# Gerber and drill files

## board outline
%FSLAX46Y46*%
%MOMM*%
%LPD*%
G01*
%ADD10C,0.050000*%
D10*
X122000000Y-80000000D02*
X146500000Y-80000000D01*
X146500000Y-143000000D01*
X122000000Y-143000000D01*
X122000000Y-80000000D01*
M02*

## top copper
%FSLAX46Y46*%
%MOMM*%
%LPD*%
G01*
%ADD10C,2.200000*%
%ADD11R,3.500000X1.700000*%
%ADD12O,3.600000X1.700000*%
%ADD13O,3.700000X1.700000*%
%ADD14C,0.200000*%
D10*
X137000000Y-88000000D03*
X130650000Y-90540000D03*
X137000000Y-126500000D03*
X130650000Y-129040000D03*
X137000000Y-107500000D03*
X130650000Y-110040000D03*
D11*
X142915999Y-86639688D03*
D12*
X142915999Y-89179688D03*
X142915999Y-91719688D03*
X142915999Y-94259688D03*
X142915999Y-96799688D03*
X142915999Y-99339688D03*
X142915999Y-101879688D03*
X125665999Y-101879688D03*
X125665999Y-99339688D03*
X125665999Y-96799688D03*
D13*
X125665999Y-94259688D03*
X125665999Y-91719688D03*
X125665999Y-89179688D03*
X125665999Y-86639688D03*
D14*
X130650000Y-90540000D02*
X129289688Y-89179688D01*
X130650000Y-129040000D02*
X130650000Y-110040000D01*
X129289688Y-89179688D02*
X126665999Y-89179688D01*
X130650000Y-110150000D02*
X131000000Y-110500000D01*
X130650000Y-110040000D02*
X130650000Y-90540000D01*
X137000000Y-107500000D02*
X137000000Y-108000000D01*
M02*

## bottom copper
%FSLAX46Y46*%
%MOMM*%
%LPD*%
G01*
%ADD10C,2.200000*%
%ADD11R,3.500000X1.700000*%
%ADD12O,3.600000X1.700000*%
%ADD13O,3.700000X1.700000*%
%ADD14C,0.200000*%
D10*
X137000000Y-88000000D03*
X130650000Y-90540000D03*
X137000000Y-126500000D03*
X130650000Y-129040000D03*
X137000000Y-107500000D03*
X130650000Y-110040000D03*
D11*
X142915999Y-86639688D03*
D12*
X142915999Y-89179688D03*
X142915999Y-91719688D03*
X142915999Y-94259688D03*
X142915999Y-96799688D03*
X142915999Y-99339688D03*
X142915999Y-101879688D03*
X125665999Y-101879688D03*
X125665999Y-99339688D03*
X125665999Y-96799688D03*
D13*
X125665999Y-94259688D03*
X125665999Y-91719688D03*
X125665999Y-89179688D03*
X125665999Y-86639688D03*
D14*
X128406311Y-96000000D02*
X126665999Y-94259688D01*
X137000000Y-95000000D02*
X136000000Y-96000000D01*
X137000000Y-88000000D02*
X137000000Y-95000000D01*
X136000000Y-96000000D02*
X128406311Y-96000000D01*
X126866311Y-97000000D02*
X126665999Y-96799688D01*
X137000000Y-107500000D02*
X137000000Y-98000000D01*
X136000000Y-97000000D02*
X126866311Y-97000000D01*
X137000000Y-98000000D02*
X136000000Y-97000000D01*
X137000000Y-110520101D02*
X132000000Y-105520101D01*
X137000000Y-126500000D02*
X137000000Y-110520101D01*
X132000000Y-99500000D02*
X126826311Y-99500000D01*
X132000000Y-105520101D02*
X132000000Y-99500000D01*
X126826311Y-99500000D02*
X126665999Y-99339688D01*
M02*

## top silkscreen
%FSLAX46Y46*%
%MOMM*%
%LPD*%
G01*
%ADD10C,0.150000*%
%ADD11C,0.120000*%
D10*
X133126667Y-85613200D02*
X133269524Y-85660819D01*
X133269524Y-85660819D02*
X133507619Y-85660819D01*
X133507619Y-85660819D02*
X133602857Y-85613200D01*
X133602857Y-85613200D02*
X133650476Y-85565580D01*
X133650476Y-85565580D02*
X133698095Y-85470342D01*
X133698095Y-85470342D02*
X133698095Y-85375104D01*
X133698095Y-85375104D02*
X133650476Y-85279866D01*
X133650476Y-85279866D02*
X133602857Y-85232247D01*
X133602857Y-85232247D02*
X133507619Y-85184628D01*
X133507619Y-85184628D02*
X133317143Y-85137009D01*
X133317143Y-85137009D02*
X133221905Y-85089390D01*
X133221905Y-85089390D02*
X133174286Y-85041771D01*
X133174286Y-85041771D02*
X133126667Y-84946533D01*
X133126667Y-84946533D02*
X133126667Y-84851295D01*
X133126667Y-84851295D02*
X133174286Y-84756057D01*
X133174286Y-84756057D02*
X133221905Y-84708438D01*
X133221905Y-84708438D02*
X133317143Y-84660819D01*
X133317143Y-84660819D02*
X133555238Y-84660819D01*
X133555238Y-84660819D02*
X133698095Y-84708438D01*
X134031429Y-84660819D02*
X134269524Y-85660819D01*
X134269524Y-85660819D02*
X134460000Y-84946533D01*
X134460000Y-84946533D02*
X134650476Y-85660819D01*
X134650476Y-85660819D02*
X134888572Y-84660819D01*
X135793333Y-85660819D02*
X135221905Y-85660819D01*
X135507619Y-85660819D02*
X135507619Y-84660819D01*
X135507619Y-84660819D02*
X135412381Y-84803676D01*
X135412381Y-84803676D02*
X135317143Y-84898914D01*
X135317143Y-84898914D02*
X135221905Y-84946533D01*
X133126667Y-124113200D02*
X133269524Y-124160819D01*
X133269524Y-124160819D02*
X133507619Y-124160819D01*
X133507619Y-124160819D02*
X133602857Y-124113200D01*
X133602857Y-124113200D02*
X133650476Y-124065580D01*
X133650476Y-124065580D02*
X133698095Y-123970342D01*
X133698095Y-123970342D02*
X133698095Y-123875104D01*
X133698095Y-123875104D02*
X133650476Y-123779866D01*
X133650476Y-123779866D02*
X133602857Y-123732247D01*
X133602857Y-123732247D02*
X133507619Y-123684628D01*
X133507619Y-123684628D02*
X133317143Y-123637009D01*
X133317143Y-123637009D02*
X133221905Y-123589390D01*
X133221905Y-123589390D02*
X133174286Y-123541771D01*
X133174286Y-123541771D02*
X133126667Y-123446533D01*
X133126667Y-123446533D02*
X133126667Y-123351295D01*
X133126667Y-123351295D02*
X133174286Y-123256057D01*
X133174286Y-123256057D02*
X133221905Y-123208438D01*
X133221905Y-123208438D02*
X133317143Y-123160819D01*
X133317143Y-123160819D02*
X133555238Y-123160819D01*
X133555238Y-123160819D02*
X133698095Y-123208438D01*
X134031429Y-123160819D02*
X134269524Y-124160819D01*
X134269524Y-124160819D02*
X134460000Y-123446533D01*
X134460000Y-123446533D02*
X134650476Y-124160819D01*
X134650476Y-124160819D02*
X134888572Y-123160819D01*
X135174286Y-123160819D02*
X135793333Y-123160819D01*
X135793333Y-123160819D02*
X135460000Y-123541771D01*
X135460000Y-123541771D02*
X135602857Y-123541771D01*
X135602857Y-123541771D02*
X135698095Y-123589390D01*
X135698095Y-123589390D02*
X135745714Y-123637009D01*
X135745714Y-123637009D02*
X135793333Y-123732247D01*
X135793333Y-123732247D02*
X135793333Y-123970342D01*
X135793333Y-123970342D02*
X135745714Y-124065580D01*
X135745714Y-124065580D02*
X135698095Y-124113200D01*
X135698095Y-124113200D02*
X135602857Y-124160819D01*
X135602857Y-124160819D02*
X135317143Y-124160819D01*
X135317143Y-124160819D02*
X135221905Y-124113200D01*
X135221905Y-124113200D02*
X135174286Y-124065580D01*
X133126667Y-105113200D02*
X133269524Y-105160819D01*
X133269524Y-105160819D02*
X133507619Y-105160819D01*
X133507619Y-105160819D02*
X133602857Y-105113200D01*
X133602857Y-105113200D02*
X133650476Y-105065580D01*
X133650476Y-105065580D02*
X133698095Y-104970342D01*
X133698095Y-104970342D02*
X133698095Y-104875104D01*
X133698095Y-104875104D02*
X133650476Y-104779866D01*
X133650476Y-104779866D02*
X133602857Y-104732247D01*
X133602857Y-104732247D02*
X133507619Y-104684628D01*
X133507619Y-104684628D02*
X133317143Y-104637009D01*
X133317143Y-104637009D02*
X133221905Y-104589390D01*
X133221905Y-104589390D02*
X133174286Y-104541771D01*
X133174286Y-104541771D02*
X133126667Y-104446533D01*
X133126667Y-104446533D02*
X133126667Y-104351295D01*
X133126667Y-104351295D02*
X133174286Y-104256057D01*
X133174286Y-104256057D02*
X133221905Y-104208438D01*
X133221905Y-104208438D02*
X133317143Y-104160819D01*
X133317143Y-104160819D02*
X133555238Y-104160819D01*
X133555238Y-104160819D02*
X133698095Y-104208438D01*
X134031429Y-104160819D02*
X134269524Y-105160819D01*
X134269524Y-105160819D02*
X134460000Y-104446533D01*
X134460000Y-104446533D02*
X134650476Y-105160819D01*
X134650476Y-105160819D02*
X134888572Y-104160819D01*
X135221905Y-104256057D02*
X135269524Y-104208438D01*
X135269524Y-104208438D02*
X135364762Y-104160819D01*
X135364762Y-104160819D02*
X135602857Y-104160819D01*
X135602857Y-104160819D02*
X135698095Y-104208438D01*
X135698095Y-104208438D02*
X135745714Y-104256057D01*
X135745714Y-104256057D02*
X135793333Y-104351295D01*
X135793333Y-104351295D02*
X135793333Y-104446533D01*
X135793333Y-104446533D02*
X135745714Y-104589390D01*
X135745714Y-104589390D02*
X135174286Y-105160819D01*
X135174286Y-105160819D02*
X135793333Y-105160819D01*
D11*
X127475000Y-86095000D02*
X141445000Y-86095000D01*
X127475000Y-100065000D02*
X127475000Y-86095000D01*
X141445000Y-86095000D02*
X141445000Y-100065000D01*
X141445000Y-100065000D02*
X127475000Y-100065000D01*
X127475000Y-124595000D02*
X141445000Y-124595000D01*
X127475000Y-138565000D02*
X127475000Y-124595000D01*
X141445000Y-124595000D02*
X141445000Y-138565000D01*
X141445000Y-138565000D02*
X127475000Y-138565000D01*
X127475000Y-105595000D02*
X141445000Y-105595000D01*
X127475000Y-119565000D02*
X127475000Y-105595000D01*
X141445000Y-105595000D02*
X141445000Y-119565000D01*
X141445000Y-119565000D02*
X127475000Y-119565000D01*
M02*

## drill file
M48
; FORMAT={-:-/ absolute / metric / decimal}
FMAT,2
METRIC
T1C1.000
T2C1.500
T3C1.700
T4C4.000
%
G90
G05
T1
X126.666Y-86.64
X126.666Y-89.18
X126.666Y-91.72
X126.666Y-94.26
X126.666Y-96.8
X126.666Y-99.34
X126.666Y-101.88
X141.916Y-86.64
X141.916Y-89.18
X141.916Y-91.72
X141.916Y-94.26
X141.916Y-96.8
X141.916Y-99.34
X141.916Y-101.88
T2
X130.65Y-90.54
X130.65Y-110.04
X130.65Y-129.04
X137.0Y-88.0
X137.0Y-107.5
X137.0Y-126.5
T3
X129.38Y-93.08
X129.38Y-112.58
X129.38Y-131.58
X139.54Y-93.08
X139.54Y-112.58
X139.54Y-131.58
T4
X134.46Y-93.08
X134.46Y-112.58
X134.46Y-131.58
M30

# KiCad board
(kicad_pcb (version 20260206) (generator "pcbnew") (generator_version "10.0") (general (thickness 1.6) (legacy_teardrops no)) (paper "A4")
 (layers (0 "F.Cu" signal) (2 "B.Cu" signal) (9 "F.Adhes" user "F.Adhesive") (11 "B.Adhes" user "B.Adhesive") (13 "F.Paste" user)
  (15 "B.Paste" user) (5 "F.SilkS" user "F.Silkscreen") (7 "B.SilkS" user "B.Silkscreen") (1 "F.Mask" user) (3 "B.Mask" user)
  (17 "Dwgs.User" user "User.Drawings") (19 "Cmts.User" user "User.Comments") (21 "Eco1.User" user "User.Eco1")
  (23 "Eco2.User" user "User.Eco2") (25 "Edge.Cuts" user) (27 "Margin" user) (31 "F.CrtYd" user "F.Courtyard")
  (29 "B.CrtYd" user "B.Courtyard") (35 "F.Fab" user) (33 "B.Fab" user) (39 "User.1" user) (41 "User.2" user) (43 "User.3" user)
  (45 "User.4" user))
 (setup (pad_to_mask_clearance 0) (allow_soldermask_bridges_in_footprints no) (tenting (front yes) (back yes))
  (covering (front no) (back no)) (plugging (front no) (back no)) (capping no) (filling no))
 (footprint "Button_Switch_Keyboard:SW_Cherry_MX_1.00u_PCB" (layer "F.Cu") (at 137 88)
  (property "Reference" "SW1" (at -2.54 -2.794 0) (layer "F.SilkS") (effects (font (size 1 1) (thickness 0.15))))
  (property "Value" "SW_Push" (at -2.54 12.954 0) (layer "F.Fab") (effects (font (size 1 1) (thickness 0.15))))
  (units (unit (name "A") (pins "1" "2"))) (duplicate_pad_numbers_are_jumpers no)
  (fp_line (start -9.525 -1.905) (end 4.445 -1.905) (stroke (width 0.12) (type solid)) (layer "F.SilkS"))
  (fp_line (start -9.525 12.065) (end -9.525 -1.905) (stroke (width 0.12) (type solid)) (layer "F.SilkS"))
  (fp_line (start 4.445 -1.905) (end 4.445 12.065) (stroke (width 0.12) (type solid)) (layer "F.SilkS"))
  (fp_line (start 4.445 12.065) (end -9.525 12.065) (stroke (width 0.12) (type solid)) (layer "F.SilkS"))
  (pad "" np_thru_hole circle (at -7.62 5.08) (size 1.7 1.7) (drill 1.7) (layers "*.Cu" "*.Mask"))
  (pad "" np_thru_hole circle (at -2.54 5.08) (size 4 4) (drill 4) (layers "*.Cu" "*.Mask"))
  (pad "" np_thru_hole circle (at 2.54 5.08) (size 1.7 1.7) (drill 1.7) (layers "*.Cu" "*.Mask"))
  (pad "1" thru_hole circle (at 0 0) (size 2.2 2.2) (drill 1.5) (layers "*.Cu" "*.Mask") (remove_unused_layers no)
   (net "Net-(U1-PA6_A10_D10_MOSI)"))
  (pad "2" thru_hole circle (at -6.35 2.54) (size 2.2 2.2) (drill 1.5) (layers "*.Cu" "*.Mask") (remove_unused_layers no) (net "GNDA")))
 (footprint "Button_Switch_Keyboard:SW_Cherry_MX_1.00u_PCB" (layer "F.Cu") (at 137 126.5)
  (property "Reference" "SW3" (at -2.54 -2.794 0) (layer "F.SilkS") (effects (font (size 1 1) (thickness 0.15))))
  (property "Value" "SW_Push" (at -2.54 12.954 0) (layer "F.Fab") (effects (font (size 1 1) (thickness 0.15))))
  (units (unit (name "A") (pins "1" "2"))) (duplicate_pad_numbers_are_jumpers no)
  (fp_line (start -9.525 -1.905) (end 4.445 -1.905) (stroke (width 0.12) (type solid)) (layer "F.SilkS"))
  (fp_line (start -9.525 12.065) (end -9.525 -1.905) (stroke (width 0.12) (type solid)) (layer "F.SilkS"))
  (fp_line (start 4.445 -1.905) (end 4.445 12.065) (stroke (width 0.12) (type solid)) (layer "F.SilkS"))
  (fp_line (start 4.445 12.065) (end -9.525 12.065) (stroke (width 0.12) (type solid)) (layer "F.SilkS"))
  (pad "" np_thru_hole circle (at -7.62 5.08) (size 1.7 1.7) (drill 1.7) (layers "*.Cu" "*.Mask"))
  (pad "" np_thru_hole circle (at -2.54 5.08) (size 4 4) (drill 4) (layers "*.Cu" "*.Mask"))
  (pad "" np_thru_hole circle (at 2.54 5.08) (size 1.7 1.7) (drill 1.7) (layers "*.Cu" "*.Mask"))
  (pad "1" thru_hole circle (at 0 0) (size 2.2 2.2) (drill 1.5) (layers "*.Cu" "*.Mask") (remove_unused_layers no)
   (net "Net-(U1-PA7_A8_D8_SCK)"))
  (pad "2" thru_hole circle (at -6.35 2.54) (size 2.2 2.2) (drill 1.5) (layers "*.Cu" "*.Mask") (remove_unused_layers no) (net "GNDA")))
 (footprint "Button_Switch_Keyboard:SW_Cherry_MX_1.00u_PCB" (layer "F.Cu") (at 137 107.5)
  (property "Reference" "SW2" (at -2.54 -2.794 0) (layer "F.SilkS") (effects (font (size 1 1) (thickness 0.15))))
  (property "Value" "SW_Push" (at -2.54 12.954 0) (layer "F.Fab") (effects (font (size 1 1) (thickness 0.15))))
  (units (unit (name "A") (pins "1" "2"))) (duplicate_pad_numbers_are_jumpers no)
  (fp_line (start -9.525 -1.905) (end 4.445 -1.905) (stroke (width 0.12) (type solid)) (layer "F.SilkS"))
  (fp_line (start -9.525 12.065) (end -9.525 -1.905) (stroke (width 0.12) (type solid)) (layer "F.SilkS"))
  (fp_line (start 4.445 -1.905) (end 4.445 12.065) (stroke (width 0.12) (type solid)) (layer "F.SilkS"))
  (fp_line (start 4.445 12.065) (end -9.525 12.065) (stroke (width 0.12) (type solid)) (layer "F.SilkS"))
  (pad "" np_thru_hole circle (at -7.62 5.08) (size 1.7 1.7) (drill 1.7) (layers "*.Cu" "*.Mask"))
  (pad "" np_thru_hole circle (at -2.54 5.08) (size 4 4) (drill 4) (layers "*.Cu" "*.Mask"))
  (pad "" np_thru_hole circle (at 2.54 5.08) (size 1.7 1.7) (drill 1.7) (layers "*.Cu" "*.Mask"))
  (pad "1" thru_hole circle (at 0 0) (size 2.2 2.2) (drill 1.5) (layers "*.Cu" "*.Mask") (remove_unused_layers no)
   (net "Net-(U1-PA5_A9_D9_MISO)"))
  (pad "2" thru_hole circle (at -6.35 2.54) (size 2.2 2.2) (drill 1.5) (layers "*.Cu" "*.Mask") (remove_unused_layers no) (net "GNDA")))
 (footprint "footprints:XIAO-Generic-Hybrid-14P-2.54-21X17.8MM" (layer "B.Cu") (at 134.290999 94.259688 180)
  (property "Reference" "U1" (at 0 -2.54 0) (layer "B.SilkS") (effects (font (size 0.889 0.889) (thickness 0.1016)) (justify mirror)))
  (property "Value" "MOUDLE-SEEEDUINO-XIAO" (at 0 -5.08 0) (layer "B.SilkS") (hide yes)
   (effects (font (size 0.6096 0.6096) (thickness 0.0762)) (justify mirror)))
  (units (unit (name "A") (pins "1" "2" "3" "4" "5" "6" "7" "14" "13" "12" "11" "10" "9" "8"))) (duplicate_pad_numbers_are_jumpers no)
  (pad "1" thru_hole rect (at -7.625 7.62 180) (size 3.5 1.7) (drill 1 (offset -1 0)) (layers "*.Cu" "*.Mask") (remove_unused_layers no)
   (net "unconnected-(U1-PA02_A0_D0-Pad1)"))
  (pad "2" thru_hole oval (at -7.625 5.08 180) (size 3.6 1.7) (drill 1 (offset -1 0)) (layers "*.Cu" "*.Mask") (remove_unused_layers no)
   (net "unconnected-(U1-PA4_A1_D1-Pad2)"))
  (pad "3" thru_hole oval (at -7.625 2.54 180) (size 3.6 1.7) (drill 1 (offset -1 0)) (layers "*.Cu" "*.Mask") (remove_unused_layers no)
   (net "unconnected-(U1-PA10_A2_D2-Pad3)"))
  (pad "4" thru_hole oval (at -7.625 0 180) (size 3.6 1.7) (drill 1 (offset -1 0)) (layers "*.Cu" "*.Mask") (remove_unused_layers no)
   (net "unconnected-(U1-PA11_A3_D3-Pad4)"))
  (pad "5" thru_hole oval (at -7.625 -2.54 180) (size 3.6 1.7) (drill 1 (offset -1 0)) (layers "*.Cu" "*.Mask") (remove_unused_layers no)
   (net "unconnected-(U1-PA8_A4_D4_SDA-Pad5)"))
  (pad "6" thru_hole oval (at -7.625 -5.08) (size 3.6 1.7) (drill 1 (offset 1 0)) (layers "*.Cu" "*.Mask") (remove_unused_layers no)
   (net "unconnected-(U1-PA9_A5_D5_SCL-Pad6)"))
  (pad "7" thru_hole oval (at -7.625 -7.62 180) (size 3.6 1.7) (drill 1 (offset -1 0)) (layers "*.Cu" "*.Mask") (remove_unused_layers no)
   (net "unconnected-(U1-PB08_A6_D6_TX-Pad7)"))
  (pad "8" thru_hole oval (at 7.625 -7.62 180) (size 3.6 1.7) (drill 1 (offset 1 0)) (layers "*.Cu" "*.Mask") (remove_unused_layers no)
   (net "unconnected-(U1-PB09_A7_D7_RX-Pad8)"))
  (pad "9" thru_hole oval (at 7.625 -5.08 180) (size 3.6 1.7) (drill 1 (offset 1 0)) (layers "*.Cu" "*.Mask") (remove_unused_layers no)
   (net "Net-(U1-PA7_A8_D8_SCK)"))
  (pad "10" thru_hole oval (at 7.625 -2.54 180) (size 3.6 1.7) (drill 1 (offset 1 0)) (layers "*.Cu" "*.Mask") (remove_unused_layers no)
   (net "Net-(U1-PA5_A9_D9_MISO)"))
  (pad "11" thru_hole oval (at 7.625 0 180) (size 3.7 1.7) (drill 1 (offset 1 0)) (layers "*.Cu" "*.Mask") (remove_unused_layers no)
   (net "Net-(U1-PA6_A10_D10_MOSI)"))
  (pad "12" thru_hole oval (at 7.625 2.54 180) (size 3.7 1.7) (drill 1 (offset 1 0)) (layers "*.Cu" "*.Mask") (remove_unused_layers no)
   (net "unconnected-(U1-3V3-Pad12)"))
  (pad "13" thru_hole oval (at 7.625 5.08 180) (size 3.7 1.7) (drill 1 (offset 1 0)) (layers "*.Cu" "*.Mask") (remove_unused_layers no)
   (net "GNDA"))
  (pad "14" thru_hole oval (at 7.625 7.62 180) (size 3.7 1.7) (drill 1 (offset 1 0)) (layers "*.Cu" "*.Mask") (remove_unused_layers no)
   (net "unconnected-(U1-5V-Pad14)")))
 (gr_rect (start 122 80) (end 146.5 143) (stroke (width 0.05) (type default)) (fill no) (layer "Edge.Cuts"))
 (segment (start 128.406311 96) (end 126.665999 94.259688) (width 0.2) (layer "B.Cu") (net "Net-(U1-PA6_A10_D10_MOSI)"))
 (segment (start 137 95) (end 136 96) (width 0.2) (layer "B.Cu") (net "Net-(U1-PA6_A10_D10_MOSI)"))
 (segment (start 137 88) (end 137 95) (width 0.2) (layer "B.Cu") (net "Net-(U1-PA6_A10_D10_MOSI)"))
 (segment (start 136 96) (end 128.406311 96) (width 0.2) (layer "B.Cu") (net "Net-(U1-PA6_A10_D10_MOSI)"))
 (segment (start 130.65 90.54) (end 129.289688 89.179688) (width 0.2) (layer "F.Cu") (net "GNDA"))
 (segment (start 130.65 129.04) (end 130.65 110.04) (width 0.2) (layer "F.Cu") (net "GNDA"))
 (segment (start 129.289688 89.179688) (end 126.665999 89.179688) (width 0.2) (layer "F.Cu") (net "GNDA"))
 (segment (start 130.65 110.15) (end 131 110.5) (width 0.2) (layer "F.Cu") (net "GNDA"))
 (segment (start 130.65 110.04) (end 130.65 90.54) (width 0.2) (layer "F.Cu") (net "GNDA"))
 (segment (start 137 107.5) (end 137 108) (width 0.2) (layer "F.Cu") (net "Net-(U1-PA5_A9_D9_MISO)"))
 (segment (start 126.866311 97) (end 126.665999 96.799688) (width 0.2) (layer "B.Cu") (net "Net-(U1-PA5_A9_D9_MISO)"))
 (segment (start 137 107.5) (end 137 98) (width 0.2) (layer "B.Cu") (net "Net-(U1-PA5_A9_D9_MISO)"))
 (segment (start 136 97) (end 126.866311 97) (width 0.2) (layer "B.Cu") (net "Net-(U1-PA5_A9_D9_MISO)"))
 (segment (start 137 98) (end 136 97) (width 0.2) (layer "B.Cu") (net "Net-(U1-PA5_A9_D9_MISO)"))
 (segment (start 137 110.520101) (end 132 105.520101) (width 0.2) (layer "B.Cu") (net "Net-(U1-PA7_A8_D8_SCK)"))
 (segment (start 137 126.5) (end 137 110.520101) (width 0.2) (layer "B.Cu") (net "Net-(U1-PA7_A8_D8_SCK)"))
 (segment (start 132 99.5) (end 126.826311 99.5) (width 0.2) (layer "B.Cu") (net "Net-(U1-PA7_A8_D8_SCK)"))
 (segment (start 132 105.520101) (end 132 99.5) (width 0.2) (layer "B.Cu") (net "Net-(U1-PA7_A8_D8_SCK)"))
 (segment (start 126.826311 99.5) (end 126.665999 99.339688) (width 0.2) (layer "B.Cu") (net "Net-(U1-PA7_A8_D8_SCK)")))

